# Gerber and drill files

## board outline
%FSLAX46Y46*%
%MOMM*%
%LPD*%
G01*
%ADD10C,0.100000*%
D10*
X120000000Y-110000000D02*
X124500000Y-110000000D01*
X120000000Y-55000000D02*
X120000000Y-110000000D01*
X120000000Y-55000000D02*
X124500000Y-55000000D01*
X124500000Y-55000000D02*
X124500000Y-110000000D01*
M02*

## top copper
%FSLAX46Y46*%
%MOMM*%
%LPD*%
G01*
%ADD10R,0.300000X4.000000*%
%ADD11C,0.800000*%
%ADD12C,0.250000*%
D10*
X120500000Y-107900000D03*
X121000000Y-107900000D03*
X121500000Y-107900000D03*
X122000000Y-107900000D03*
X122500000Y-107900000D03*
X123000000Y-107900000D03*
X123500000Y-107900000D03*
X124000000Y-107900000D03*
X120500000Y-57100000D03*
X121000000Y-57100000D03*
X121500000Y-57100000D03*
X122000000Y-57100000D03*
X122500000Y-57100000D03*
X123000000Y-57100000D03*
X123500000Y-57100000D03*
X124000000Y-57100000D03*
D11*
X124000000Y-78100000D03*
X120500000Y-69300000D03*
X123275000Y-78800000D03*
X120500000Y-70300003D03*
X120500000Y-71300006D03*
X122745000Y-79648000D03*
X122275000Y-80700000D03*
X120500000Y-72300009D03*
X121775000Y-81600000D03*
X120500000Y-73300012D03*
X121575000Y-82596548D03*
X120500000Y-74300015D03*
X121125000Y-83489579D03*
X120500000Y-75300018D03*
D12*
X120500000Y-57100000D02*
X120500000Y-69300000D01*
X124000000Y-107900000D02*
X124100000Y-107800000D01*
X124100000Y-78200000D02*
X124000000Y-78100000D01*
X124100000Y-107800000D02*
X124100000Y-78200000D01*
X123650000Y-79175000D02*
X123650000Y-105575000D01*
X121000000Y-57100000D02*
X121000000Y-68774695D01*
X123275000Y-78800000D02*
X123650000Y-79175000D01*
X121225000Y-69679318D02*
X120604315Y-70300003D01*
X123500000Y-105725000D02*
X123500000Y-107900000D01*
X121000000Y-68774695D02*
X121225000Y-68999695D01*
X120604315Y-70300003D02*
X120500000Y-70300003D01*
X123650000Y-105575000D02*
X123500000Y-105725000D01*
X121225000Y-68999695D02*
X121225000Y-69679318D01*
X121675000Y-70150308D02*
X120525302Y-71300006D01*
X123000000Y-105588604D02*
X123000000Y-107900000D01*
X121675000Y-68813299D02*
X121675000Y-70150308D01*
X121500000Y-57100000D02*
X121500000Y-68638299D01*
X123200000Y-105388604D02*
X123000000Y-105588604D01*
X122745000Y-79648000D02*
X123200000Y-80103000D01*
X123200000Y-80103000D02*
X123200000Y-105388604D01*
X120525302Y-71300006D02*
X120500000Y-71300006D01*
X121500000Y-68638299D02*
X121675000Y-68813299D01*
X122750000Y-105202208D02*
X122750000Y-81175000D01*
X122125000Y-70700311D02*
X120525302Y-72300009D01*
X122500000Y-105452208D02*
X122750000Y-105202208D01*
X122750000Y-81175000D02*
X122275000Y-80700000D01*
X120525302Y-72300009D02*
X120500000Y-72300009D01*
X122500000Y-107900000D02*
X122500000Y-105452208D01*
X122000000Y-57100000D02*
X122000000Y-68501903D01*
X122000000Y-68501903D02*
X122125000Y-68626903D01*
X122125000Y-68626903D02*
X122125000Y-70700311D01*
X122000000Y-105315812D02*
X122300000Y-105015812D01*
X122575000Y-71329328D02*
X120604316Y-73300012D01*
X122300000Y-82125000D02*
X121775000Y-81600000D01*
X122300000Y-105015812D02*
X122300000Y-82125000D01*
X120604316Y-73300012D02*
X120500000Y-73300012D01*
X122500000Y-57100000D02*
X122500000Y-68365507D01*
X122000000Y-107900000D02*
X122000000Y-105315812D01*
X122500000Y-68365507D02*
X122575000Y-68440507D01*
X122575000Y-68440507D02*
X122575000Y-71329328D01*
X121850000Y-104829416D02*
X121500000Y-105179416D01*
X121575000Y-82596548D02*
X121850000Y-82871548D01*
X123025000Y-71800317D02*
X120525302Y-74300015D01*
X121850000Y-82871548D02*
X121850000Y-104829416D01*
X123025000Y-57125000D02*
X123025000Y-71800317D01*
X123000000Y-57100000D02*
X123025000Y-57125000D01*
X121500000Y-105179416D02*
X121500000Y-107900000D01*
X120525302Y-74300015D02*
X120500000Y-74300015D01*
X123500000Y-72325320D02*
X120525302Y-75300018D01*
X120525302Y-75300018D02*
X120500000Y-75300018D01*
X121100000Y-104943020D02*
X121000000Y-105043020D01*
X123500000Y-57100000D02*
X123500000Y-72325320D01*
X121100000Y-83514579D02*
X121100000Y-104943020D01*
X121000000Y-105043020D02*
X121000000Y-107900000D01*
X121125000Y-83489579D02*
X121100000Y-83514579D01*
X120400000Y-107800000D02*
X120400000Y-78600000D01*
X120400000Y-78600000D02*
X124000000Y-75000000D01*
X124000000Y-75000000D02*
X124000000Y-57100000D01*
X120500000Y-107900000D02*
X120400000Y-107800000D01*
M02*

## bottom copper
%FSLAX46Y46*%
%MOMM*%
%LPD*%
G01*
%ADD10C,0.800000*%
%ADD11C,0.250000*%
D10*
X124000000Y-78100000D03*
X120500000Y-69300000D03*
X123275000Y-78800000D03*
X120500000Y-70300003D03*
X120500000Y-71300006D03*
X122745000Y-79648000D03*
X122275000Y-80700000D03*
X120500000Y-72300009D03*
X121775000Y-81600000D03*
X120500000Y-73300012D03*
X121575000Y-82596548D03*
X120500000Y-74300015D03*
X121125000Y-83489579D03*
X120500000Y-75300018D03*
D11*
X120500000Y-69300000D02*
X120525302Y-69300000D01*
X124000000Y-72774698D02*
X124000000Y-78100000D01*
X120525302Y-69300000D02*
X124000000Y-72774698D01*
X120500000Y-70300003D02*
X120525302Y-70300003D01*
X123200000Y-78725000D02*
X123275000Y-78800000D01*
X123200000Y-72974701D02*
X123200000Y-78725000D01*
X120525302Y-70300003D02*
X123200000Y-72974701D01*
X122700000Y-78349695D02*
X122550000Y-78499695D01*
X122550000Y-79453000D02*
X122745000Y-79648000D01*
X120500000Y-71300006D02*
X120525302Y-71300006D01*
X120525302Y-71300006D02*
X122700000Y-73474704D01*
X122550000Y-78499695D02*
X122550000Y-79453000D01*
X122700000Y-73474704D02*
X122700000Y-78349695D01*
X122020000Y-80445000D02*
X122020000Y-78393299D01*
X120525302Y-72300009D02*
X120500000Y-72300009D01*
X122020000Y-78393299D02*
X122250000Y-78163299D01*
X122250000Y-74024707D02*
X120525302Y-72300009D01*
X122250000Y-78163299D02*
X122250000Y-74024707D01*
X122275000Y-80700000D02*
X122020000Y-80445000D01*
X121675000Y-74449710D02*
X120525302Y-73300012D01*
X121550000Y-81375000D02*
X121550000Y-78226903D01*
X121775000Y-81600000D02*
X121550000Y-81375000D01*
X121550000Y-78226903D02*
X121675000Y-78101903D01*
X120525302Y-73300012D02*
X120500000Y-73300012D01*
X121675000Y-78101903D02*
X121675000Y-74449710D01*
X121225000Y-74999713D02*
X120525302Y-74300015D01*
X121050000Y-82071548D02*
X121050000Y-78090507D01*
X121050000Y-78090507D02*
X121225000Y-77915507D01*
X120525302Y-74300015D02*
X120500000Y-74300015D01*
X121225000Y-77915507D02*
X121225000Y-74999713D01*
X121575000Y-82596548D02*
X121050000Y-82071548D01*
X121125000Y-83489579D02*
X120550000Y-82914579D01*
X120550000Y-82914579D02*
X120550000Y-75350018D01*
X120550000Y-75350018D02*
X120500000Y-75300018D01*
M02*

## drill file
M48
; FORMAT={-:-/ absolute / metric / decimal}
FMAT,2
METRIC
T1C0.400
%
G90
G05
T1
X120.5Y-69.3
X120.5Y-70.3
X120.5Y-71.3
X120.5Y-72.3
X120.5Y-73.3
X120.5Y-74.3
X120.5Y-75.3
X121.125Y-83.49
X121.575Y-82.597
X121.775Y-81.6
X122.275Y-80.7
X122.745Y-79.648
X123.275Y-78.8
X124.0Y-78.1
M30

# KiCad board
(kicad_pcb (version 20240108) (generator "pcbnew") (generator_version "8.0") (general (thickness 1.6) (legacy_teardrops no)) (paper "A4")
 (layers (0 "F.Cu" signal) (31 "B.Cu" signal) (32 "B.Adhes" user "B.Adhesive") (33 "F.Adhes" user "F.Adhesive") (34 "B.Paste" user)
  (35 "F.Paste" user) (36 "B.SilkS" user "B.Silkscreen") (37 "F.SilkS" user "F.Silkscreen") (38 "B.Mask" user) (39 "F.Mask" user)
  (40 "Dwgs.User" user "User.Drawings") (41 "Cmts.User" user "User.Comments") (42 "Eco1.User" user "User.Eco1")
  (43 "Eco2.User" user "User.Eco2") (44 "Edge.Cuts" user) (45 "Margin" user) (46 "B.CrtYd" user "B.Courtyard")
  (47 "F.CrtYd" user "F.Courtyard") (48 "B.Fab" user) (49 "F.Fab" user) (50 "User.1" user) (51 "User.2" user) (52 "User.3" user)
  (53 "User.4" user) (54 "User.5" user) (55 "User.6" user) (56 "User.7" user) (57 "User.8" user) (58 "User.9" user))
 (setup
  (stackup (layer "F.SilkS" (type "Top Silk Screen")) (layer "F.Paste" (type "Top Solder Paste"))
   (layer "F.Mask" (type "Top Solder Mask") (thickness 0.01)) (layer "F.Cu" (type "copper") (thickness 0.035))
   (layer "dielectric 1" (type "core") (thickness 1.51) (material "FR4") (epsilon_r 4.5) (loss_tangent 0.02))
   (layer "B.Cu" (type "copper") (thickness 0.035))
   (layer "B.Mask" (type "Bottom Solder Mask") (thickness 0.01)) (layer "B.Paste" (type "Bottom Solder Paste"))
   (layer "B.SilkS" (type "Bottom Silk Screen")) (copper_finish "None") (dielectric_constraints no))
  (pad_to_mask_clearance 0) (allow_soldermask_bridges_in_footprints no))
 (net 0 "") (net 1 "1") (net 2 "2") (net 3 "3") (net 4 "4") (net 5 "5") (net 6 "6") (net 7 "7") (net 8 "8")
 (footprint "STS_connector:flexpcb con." (layer "F.Cu") (at 120 109.9)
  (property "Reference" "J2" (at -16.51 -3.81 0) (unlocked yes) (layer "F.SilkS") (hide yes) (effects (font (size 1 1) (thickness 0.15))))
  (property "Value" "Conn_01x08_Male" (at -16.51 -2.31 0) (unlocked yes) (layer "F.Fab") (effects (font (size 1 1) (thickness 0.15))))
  (pad "1" smd rect (at 0.5 -2) (size 0.3 4) (layers "F.Cu" "F.Paste" "F.Mask") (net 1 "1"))
  (pad "2" smd rect (at 1 -2) (size 0.3 4) (layers "F.Cu" "F.Paste" "F.Mask") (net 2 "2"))
  (pad "3" smd rect (at 1.5 -2) (size 0.3 4) (layers "F.Cu" "F.Paste" "F.Mask") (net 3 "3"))
  (pad "4" smd rect (at 2 -2) (size 0.3 4) (layers "F.Cu" "F.Paste" "F.Mask") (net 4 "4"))
  (pad "5" smd rect (at 2.5 -2) (size 0.3 4) (layers "F.Cu" "F.Paste" "F.Mask") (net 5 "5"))
  (pad "6" smd rect (at 3 -2) (size 0.3 4) (layers "F.Cu" "F.Paste" "F.Mask") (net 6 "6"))
  (pad "7" smd rect (at 3.5 -2) (size 0.3 4) (layers "F.Cu" "F.Paste" "F.Mask") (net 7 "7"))
  (pad "8" smd rect (at 4 -2) (size 0.3 4) (layers "F.Cu" "F.Paste" "F.Mask") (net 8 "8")))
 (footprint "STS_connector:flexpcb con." (layer "F.Cu") (at 120 59.1)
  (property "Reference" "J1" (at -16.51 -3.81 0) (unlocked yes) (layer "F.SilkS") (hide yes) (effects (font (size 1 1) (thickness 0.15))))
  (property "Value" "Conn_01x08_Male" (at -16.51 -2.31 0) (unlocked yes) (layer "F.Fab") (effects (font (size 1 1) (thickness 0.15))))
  (pad "1" smd rect (at 0.5 -2) (size 0.3 4) (layers "F.Cu" "F.Paste" "F.Mask") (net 8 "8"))
  (pad "2" smd rect (at 1 -2) (size 0.3 4) (layers "F.Cu" "F.Paste" "F.Mask") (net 7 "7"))
  (pad "3" smd rect (at 1.5 -2) (size 0.3 4) (layers "F.Cu" "F.Paste" "F.Mask") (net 6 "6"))
  (pad "4" smd rect (at 2 -2) (size 0.3 4) (layers "F.Cu" "F.Paste" "F.Mask") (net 5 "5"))
  (pad "5" smd rect (at 2.5 -2) (size 0.3 4) (layers "F.Cu" "F.Paste" "F.Mask") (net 4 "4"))
  (pad "6" smd rect (at 3 -2) (size 0.3 4) (layers "F.Cu" "F.Paste" "F.Mask") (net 3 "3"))
  (pad "7" smd rect (at 3.5 -2) (size 0.3 4) (layers "F.Cu" "F.Paste" "F.Mask") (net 2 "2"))
  (pad "8" smd rect (at 4 -2) (size 0.3 4) (layers "F.Cu" "F.Paste" "F.Mask") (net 1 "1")))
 (gr_line (start 120 110) (end 124.5 110) (stroke (width 0.1) (type solid)) (layer "Edge.Cuts"))
 (gr_line (start 120 55) (end 120 110) (stroke (width 0.1) (type solid)) (layer "Edge.Cuts"))
 (gr_line (start 120 55) (end 124.5 55) (stroke (width 0.1) (type solid)) (layer "Edge.Cuts"))
 (gr_line (start 124.5 55) (end 124.5 110) (stroke (width 0.1) (type solid)) (layer "Edge.Cuts"))
 (segment (start 120.5 57.1) (end 120.5 69.3) (width 0.25) (layer "F.Cu") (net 8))
 (segment (start 124 107.9) (end 124.1 107.8) (width 0.25) (layer "F.Cu") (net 8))
 (segment (start 124.1 78.2) (end 124 78.1) (width 0.25) (layer "F.Cu") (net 8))
 (segment (start 124.1 107.8) (end 124.1 78.2) (width 0.25) (layer "F.Cu") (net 8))
 (via (at 124 78.1) (size 0.8) (drill 0.4) (layers "F.Cu" "B.Cu") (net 8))
 (via (at 120.5 69.3) (size 0.8) (drill 0.4) (layers "F.Cu" "B.Cu") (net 8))
 (segment (start 120.5 69.3) (end 120.525302 69.3) (width 0.25) (layer "B.Cu") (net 8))
 (segment (start 124 72.774698) (end 124 78.1) (width 0.25) (layer "B.Cu") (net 8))
 (segment (start 120.525302 69.3) (end 124 72.774698) (width 0.25) (layer "B.Cu") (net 8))
 (segment (start 123.65 79.175) (end 123.65 105.575) (width 0.25) (layer "F.Cu") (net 7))
 (segment (start 121 57.1) (end 121 68.774695) (width 0.25) (layer "F.Cu") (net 7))
 (segment (start 123.275 78.8) (end 123.65 79.175) (width 0.25) (layer "F.Cu") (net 7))
 (segment (start 121.225 69.679318) (end 120.604315 70.300003) (width 0.25) (layer "F.Cu") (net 7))
 (segment (start 123.5 105.725) (end 123.5 107.9) (width 0.25) (layer "F.Cu") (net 7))
 (segment (start 121 68.774695) (end 121.225 68.999695) (width 0.25) (layer "F.Cu") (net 7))
 (segment (start 120.604315 70.300003) (end 120.5 70.300003) (width 0.25) (layer "F.Cu") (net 7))
 (segment (start 123.65 105.575) (end 123.5 105.725) (width 0.25) (layer "F.Cu") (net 7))
 (segment (start 121.225 68.999695) (end 121.225 69.679318) (width 0.25) (layer "F.Cu") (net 7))
 (via (at 123.275 78.8) (size 0.8) (drill 0.4) (layers "F.Cu" "B.Cu") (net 7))
 (via (at 120.5 70.300003) (size 0.8) (drill 0.4) (layers "F.Cu" "B.Cu") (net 7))
 (segment (start 120.5 70.300003) (end 120.525302 70.300003) (width 0.25) (layer "B.Cu") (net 7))
 (segment (start 123.2 78.725) (end 123.275 78.8) (width 0.25) (layer "B.Cu") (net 7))
 (segment (start 123.2 72.974701) (end 123.2 78.725) (width 0.25) (layer "B.Cu") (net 7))
 (segment (start 120.525302 70.300003) (end 123.2 72.974701) (width 0.25) (layer "B.Cu") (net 7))
 (segment (start 121.675 70.150308) (end 120.525302 71.300006) (width 0.25) (layer "F.Cu") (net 6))
 (segment (start 123 105.588604) (end 123 107.9) (width 0.25) (layer "F.Cu") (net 6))
 (segment (start 121.675 68.813299) (end 121.675 70.150308) (width 0.25) (layer "F.Cu") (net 6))
 (segment (start 121.5 57.1) (end 121.5 68.638299) (width 0.25) (layer "F.Cu") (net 6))
 (segment (start 123.2 105.388604) (end 123 105.588604) (width 0.25) (layer "F.Cu") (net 6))
 (segment (start 122.745 79.648) (end 123.2 80.103) (width 0.25) (layer "F.Cu") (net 6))
 (segment (start 123.2 80.103) (end 123.2 105.388604) (width 0.25) (layer "F.Cu") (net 6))
 (segment (start 120.525302 71.300006) (end 120.5 71.300006) (width 0.25) (layer "F.Cu") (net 6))
 (segment (start 121.5 68.638299) (end 121.675 68.813299) (width 0.25) (layer "F.Cu") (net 6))
 (via (at 120.5 71.300006) (size 0.8) (drill 0.4) (layers "F.Cu" "B.Cu") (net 6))
 (via (at 122.745 79.648) (size 0.8) (drill 0.4) (layers "F.Cu" "B.Cu") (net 6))
 (segment (start 122.7 78.349695) (end 122.55 78.499695) (width 0.25) (layer "B.Cu") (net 6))
 (segment (start 122.55 79.453) (end 122.745 79.648) (width 0.25) (layer "B.Cu") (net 6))
 (segment (start 120.5 71.300006) (end 120.525302 71.300006) (width 0.25) (layer "B.Cu") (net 6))
 (segment (start 120.525302 71.300006) (end 122.7 73.474704) (width 0.25) (layer "B.Cu") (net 6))
 (segment (start 122.55 78.499695) (end 122.55 79.453) (width 0.25) (layer "B.Cu") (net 6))
 (segment (start 122.7 73.474704) (end 122.7 78.349695) (width 0.25) (layer "B.Cu") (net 6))
 (segment (start 122.75 105.202208) (end 122.75 81.175) (width 0.25) (layer "F.Cu") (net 5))
 (segment (start 122.125 70.700311) (end 120.525302 72.300009) (width 0.25) (layer "F.Cu") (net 5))
 (segment (start 122.5 105.452208) (end 122.75 105.202208) (width 0.25) (layer "F.Cu") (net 5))
 (segment (start 122.75 81.175) (end 122.275 80.7) (width 0.25) (layer "F.Cu") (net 5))
 (segment (start 120.525302 72.300009) (end 120.5 72.300009) (width 0.25) (layer "F.Cu") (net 5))
 (segment (start 122.5 107.9) (end 122.5 105.452208) (width 0.25) (layer "F.Cu") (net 5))
 (segment (start 122 57.1) (end 122 68.501903) (width 0.25) (layer "F.Cu") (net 5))
 (segment (start 122 68.501903) (end 122.125 68.626903) (width 0.25) (layer "F.Cu") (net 5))
 (segment (start 122.125 68.626903) (end 122.125 70.700311) (width 0.25) (layer "F.Cu") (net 5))
 (via (at 122.275 80.7) (size 0.8) (drill 0.4) (layers "F.Cu" "B.Cu") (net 5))
 (via (at 120.5 72.300009) (size 0.8) (drill 0.4) (layers "F.Cu" "B.Cu") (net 5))
 (segment (start 122.02 80.445) (end 122.02 78.393299) (width 0.25) (layer "B.Cu") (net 5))
 (segment (start 120.525302 72.300009) (end 120.5 72.300009) (width 0.25) (layer "B.Cu") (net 5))
 (segment (start 122.02 78.393299) (end 122.25 78.163299) (width 0.25) (layer "B.Cu") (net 5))
 (segment (start 122.25 74.024707) (end 120.525302 72.300009) (width 0.25) (layer "B.Cu") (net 5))
 (segment (start 122.25 78.163299) (end 122.25 74.024707) (width 0.25) (layer "B.Cu") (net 5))
 (segment (start 122.275 80.7) (end 122.02 80.445) (width 0.25) (layer "B.Cu") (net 5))
 (segment (start 122 105.315812) (end 122.3 105.015812) (width 0.25) (layer "F.Cu") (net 4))
 (segment (start 122.575 71.329328) (end 120.604316 73.300012) (width 0.25) (layer "F.Cu") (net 4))
 (segment (start 122.3 82.125) (end 121.775 81.6) (width 0.25) (layer "F.Cu") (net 4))
 (segment (start 122.3 105.015812) (end 122.3 82.125) (width 0.25) (layer "F.Cu") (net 4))
 (segment (start 120.604316 73.300012) (end 120.5 73.300012) (width 0.25) (layer "F.Cu") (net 4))
 (segment (start 122.5 57.1) (end 122.5 68.365507) (width 0.25) (layer "F.Cu") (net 4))
 (segment (start 122 107.9) (end 122 105.315812) (width 0.25) (layer "F.Cu") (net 4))
 (segment (start 122.5 68.365507) (end 122.575 68.440507) (width 0.25) (layer "F.Cu") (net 4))
 (segment (start 122.575 68.440507) (end 122.575 71.329328) (width 0.25) (layer "F.Cu") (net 4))
 (via (at 121.775 81.6) (size 0.8) (drill 0.4) (layers "F.Cu" "B.Cu") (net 4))
 (via (at 120.5 73.300012) (size 0.8) (drill 0.4) (layers "F.Cu" "B.Cu") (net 4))
 (segment (start 121.675 74.44971) (end 120.525302 73.300012) (width 0.25) (layer "B.Cu") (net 4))
 (segment (start 121.55 81.375) (end 121.55 78.226903) (width 0.25) (layer "B.Cu") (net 4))
 (segment (start 121.775 81.6) (end 121.55 81.375) (width 0.25) (layer "B.Cu") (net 4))
 (segment (start 121.55 78.226903) (end 121.675 78.101903) (width 0.25) (layer "B.Cu") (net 4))
 (segment (start 120.525302 73.300012) (end 120.5 73.300012) (width 0.25) (layer "B.Cu") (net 4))
 (segment (start 121.675 78.101903) (end 121.675 74.44971) (width 0.25) (layer "B.Cu") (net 4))
 (segment (start 121.85 104.829416) (end 121.5 105.179416) (width 0.25) (layer "F.Cu") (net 3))
 (segment (start 121.575 82.596548) (end 121.85 82.871548) (width 0.25) (layer "F.Cu") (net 3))
 (segment (start 123.025 71.800317) (end 120.525302 74.300015) (width 0.25) (layer "F.Cu") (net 3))
 (segment (start 121.85 82.871548) (end 121.85 104.829416) (width 0.25) (layer "F.Cu") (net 3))
 (segment (start 123.025 57.125) (end 123.025 71.800317) (width 0.25) (layer "F.Cu") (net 3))
 (segment (start 123 57.1) (end 123.025 57.125) (width 0.25) (layer "F.Cu") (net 3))
 (segment (start 121.5 105.179416) (end 121.5 107.9) (width 0.25) (layer "F.Cu") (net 3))
 (segment (start 120.525302 74.300015) (end 120.5 74.300015) (width 0.25) (layer "F.Cu") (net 3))
 (via (at 121.575 82.596548) (size 0.8) (drill 0.4) (layers "F.Cu" "B.Cu") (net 3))
 (via (at 120.5 74.300015) (size 0.8) (drill 0.4) (layers "F.Cu" "B.Cu") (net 3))
 (segment (start 121.225 74.999713) (end 120.525302 74.300015) (width 0.25) (layer "B.Cu") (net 3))
 (segment (start 121.05 82.071548) (end 121.05 78.090507) (width 0.25) (layer "B.Cu") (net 3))
 (segment (start 121.05 78.090507) (end 121.225 77.915507) (width 0.25) (layer "B.Cu") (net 3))
 (segment (start 120.525302 74.300015) (end 120.5 74.300015) (width 0.25) (layer "B.Cu") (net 3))
 (segment (start 121.225 77.915507) (end 121.225 74.999713) (width 0.25) (layer "B.Cu") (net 3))
 (segment (start 121.575 82.596548) (end 121.05 82.071548) (width 0.25) (layer "B.Cu") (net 3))
 (segment (start 123.5 72.32532) (end 120.525302 75.300018) (width 0.25) (layer "F.Cu") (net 2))
 (segment (start 120.525302 75.300018) (end 120.5 75.300018) (width 0.25) (layer "F.Cu") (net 2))
 (segment (start 121.1 104.94302) (end 121 105.04302) (width 0.25) (layer "F.Cu") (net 2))
 (segment (start 123.5 57.1) (end 123.5 72.32532) (width 0.25) (layer "F.Cu") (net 2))
 (segment (start 121.1 83.514579) (end 121.1 104.94302) (width 0.25) (layer "F.Cu") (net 2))
 (segment (start 121 105.04302) (end 121 107.9) (width 0.25) (layer "F.Cu") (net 2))
 (segment (start 121.125 83.489579) (end 121.1 83.514579) (width 0.25) (layer "F.Cu") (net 2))
 (via (at 121.125 83.489579) (size 0.8) (drill 0.4) (layers "F.Cu" "B.Cu") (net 2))
 (via (at 120.5 75.300018) (size 0.8) (drill 0.4) (layers "F.Cu" "B.Cu") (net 2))
 (segment (start 121.125 83.489579) (end 120.55 82.914579) (width 0.25) (layer "B.Cu") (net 2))
 (segment (start 120.55 82.914579) (end 120.55 75.350018) (width 0.25) (layer "B.Cu") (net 2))
 (segment (start 120.55 75.350018) (end 120.5 75.300018) (width 0.25) (layer "B.Cu") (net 2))
 (segment (start 120.4 107.8) (end 120.4 78.6) (width 0.25) (layer "F.Cu") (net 1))
 (segment (start 120.4 78.6) (end 124 75) (width 0.25) (layer "F.Cu") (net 1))
 (segment (start 124 75) (end 124 57.1) (width 0.25) (layer "F.Cu") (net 1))
 (segment (start 120.5 107.9) (end 120.4 107.8) (width 0.25) (layer "F.Cu") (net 1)))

